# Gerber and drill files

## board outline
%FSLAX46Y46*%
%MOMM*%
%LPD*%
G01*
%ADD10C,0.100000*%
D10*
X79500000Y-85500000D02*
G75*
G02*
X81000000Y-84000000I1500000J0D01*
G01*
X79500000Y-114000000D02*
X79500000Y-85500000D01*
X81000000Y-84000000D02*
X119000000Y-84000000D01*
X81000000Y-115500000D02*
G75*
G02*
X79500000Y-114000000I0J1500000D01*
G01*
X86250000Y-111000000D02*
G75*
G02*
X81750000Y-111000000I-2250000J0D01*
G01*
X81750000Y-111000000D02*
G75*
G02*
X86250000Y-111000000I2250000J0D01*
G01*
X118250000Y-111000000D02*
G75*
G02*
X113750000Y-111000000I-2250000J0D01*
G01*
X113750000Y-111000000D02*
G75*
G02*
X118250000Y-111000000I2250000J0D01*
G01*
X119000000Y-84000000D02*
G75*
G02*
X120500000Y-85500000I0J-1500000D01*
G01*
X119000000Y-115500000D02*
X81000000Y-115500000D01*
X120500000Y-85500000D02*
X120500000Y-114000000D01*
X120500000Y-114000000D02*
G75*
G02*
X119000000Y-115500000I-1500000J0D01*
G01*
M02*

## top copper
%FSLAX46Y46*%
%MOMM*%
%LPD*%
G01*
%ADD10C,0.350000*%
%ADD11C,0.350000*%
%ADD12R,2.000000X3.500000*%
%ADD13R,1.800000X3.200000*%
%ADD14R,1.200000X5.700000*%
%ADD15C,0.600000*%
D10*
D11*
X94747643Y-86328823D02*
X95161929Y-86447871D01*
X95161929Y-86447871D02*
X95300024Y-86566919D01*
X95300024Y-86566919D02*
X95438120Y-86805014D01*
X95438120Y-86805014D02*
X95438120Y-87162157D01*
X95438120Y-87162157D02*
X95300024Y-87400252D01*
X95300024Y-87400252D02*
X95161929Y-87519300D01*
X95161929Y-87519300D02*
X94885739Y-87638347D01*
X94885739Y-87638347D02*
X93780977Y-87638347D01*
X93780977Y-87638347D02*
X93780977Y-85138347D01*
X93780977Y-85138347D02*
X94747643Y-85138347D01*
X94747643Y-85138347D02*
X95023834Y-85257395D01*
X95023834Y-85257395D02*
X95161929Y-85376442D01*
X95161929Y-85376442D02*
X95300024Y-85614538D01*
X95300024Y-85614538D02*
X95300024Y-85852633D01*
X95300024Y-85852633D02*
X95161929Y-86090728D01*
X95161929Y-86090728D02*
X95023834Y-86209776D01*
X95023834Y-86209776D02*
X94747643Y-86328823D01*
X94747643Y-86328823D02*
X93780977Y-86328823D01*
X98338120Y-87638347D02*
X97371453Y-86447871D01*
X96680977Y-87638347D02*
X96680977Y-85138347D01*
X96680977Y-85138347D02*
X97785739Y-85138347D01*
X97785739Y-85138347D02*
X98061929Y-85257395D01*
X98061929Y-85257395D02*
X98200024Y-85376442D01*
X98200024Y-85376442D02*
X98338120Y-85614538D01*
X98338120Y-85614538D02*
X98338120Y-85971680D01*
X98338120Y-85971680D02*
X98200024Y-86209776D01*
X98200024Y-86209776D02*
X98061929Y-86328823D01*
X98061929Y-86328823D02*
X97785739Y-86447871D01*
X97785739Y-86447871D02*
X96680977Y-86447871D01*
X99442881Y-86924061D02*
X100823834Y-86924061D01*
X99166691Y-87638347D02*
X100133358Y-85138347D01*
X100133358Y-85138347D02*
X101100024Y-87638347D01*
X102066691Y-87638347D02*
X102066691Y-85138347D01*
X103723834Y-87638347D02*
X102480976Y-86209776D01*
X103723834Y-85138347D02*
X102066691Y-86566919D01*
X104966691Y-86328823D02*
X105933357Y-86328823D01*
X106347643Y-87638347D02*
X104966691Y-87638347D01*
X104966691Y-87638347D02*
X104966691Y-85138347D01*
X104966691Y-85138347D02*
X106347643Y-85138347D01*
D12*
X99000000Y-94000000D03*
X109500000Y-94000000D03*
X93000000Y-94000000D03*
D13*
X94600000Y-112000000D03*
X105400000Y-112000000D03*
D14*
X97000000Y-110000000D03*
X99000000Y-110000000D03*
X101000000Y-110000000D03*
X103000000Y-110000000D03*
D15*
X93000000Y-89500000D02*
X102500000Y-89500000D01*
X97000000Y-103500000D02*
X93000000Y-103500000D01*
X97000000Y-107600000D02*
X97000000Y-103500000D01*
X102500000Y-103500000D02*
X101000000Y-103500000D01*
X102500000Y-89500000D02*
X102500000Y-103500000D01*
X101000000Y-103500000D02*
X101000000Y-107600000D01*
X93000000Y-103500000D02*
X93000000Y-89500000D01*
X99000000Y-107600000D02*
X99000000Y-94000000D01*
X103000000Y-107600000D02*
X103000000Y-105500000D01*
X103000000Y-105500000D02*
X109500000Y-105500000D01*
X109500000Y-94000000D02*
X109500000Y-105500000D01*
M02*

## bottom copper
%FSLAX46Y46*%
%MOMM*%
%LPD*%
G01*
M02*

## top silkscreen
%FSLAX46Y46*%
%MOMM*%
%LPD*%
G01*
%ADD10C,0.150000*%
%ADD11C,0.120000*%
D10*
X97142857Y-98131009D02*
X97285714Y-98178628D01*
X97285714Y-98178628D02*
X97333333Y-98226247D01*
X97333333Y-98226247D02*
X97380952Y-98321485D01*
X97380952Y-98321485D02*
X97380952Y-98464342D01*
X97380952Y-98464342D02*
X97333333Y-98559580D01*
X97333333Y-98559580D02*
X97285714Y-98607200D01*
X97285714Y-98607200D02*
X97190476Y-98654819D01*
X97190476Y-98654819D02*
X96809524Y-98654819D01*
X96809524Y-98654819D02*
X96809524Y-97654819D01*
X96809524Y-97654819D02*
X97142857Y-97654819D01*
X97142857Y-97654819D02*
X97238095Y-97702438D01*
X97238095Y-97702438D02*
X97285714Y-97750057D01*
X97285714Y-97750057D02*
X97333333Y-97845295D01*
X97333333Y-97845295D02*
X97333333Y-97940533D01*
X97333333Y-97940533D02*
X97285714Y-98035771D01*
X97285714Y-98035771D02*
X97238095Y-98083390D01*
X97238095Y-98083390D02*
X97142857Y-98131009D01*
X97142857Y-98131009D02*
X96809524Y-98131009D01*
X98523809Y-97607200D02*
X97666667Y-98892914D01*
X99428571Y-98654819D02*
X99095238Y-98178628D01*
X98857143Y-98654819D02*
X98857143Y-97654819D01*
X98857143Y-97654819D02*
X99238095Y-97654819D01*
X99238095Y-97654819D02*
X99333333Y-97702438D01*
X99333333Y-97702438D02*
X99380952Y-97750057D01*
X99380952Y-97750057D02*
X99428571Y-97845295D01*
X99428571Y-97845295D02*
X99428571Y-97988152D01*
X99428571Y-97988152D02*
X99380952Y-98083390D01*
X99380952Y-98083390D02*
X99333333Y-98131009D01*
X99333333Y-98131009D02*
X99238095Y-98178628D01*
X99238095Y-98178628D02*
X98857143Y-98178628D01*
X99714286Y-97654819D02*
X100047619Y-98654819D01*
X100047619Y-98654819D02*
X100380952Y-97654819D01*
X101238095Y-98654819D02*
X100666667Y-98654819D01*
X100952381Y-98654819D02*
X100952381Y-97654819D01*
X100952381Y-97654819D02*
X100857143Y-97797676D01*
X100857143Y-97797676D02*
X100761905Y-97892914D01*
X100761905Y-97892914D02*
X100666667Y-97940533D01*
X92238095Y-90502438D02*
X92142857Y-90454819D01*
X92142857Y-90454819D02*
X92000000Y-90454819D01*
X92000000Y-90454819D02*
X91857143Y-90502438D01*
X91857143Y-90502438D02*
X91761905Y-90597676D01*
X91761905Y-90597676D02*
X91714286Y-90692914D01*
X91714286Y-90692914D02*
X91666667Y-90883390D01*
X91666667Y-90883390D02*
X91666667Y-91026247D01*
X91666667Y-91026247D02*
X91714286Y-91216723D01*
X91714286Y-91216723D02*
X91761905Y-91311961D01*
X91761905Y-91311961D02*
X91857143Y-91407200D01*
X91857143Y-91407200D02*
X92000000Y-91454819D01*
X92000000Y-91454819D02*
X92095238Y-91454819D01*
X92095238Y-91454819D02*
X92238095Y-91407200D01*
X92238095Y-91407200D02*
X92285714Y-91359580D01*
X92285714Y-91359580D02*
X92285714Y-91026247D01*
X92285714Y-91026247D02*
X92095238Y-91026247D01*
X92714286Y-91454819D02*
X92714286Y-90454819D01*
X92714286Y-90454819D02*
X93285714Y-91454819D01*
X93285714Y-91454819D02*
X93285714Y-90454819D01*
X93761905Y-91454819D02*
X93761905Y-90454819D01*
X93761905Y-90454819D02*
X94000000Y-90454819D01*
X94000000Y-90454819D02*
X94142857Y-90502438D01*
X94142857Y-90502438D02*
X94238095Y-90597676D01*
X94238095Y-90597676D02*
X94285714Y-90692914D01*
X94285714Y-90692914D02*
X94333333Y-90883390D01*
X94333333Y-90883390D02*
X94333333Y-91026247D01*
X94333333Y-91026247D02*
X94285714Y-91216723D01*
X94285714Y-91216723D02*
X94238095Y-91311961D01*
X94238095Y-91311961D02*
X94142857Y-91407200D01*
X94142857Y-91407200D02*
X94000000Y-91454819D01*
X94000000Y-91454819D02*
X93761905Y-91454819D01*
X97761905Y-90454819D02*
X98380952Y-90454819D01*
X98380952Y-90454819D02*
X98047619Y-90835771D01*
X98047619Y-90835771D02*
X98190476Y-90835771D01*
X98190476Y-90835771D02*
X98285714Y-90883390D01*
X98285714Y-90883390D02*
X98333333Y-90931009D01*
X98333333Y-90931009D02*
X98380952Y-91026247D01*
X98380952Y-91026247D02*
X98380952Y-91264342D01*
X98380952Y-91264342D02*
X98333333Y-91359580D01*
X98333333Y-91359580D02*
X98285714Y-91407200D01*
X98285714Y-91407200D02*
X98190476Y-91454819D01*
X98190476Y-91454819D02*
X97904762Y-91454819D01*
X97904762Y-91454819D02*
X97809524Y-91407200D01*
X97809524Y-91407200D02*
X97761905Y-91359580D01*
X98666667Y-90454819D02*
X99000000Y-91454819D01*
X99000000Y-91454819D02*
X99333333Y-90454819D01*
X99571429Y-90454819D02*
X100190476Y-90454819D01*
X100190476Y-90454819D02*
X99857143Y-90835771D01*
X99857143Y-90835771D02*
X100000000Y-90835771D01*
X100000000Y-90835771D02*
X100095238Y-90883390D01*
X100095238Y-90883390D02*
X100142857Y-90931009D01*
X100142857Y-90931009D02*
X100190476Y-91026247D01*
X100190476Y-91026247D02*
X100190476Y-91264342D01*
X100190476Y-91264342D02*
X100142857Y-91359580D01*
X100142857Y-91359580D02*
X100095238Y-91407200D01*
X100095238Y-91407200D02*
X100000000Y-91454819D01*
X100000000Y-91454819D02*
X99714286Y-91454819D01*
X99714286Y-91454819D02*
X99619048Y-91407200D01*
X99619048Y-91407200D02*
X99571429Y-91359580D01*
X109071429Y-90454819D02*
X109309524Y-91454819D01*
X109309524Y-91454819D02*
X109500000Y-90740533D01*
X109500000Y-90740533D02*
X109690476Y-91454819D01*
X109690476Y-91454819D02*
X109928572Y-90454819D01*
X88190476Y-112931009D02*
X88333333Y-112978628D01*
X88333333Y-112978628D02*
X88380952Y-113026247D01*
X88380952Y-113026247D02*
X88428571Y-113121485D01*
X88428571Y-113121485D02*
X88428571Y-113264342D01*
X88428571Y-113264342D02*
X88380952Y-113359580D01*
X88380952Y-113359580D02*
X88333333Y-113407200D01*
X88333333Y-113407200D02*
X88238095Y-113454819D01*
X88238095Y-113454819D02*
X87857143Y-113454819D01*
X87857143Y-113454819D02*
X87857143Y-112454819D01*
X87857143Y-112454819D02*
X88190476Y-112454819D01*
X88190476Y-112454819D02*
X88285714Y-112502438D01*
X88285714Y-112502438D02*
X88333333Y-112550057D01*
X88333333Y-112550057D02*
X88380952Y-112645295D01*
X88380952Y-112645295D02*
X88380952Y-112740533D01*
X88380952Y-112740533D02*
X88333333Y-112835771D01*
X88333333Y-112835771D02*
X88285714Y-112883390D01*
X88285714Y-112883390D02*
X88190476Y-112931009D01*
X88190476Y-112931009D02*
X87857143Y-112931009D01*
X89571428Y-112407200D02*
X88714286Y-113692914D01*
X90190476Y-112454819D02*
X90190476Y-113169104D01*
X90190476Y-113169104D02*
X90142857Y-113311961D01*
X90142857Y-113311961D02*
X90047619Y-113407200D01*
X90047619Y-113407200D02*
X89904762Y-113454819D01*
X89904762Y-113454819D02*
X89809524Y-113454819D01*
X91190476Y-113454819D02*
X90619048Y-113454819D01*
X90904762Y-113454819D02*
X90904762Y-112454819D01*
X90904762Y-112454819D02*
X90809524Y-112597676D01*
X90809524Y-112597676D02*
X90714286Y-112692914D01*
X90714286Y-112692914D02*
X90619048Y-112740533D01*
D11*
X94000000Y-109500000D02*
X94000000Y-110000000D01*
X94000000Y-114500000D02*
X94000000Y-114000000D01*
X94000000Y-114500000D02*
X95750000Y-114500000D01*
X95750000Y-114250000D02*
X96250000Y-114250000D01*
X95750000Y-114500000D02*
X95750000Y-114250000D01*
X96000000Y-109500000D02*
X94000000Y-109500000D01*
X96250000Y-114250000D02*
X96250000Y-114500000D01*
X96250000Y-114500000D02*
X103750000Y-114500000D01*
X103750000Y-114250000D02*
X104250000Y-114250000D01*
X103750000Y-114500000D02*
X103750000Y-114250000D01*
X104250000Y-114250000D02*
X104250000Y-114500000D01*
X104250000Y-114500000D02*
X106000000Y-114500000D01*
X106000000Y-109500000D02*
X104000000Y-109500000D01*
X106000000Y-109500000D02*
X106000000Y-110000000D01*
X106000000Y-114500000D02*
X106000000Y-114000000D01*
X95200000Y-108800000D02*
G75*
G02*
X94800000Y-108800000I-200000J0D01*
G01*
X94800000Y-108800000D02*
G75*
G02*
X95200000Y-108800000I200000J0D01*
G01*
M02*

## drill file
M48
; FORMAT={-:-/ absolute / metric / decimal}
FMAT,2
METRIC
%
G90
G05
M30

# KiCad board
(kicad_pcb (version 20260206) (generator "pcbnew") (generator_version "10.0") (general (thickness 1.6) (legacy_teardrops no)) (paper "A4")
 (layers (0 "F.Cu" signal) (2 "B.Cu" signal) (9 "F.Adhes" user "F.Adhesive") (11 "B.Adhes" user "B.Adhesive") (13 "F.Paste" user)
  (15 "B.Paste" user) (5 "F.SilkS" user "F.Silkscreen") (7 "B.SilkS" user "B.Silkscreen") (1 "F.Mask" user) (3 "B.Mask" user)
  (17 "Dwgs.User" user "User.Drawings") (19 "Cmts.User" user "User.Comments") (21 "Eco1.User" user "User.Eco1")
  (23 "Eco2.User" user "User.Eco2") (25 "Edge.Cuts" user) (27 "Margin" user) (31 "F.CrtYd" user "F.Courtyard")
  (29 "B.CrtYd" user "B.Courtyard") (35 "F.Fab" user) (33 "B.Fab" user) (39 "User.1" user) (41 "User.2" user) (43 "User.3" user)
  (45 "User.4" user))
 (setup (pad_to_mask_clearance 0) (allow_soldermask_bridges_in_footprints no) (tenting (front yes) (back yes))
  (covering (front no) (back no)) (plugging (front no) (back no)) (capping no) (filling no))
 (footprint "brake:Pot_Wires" (layer "F.Cu") (at 99 94)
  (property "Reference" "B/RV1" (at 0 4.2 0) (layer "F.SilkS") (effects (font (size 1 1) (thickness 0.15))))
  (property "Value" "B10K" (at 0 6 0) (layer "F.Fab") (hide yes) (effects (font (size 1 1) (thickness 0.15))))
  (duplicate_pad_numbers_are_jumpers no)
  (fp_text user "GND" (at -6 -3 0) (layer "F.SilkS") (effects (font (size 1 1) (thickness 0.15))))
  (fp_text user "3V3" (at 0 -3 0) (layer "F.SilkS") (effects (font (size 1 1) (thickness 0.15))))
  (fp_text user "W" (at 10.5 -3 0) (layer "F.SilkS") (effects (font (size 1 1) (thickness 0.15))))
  (pad "1" smd rect (at 0 0) (size 2 3.5) (layers "F.Cu" "F.Mask") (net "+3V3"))
  (pad "2" smd rect (at 10.5 0) (size 2 3.5) (layers "F.Cu" "F.Mask") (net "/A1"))
  (pad "3" smd rect (at -6 0) (size 2 3.5) (layers "F.Cu" "F.Mask") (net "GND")))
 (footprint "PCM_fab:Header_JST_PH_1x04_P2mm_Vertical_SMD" (layer "F.Cu") (at 98 110 90)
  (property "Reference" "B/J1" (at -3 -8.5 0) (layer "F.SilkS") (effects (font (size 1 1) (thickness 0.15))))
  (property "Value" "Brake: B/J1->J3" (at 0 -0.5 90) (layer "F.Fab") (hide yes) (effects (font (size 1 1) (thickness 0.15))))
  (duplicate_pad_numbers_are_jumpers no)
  (fp_line (start 0.5 -4) (end 0 -4) (stroke (width 0.12) (type solid)) (layer "F.SilkS"))
  (fp_line (start -4.5 -4) (end -4 -4) (stroke (width 0.12) (type solid)) (layer "F.SilkS"))
  (fp_line (start -4.5 -4) (end -4.5 -2.25) (stroke (width 0.12) (type solid)) (layer "F.SilkS"))
  (fp_line (start -4.25 -2.25) (end -4.25 -1.75) (stroke (width 0.12) (type solid)) (layer "F.SilkS"))
  (fp_line (start -4.5 -2.25) (end -4.25 -2.25) (stroke (width 0.12) (type solid)) (layer "F.SilkS"))
  (fp_line (start 0.5 -2) (end 0.5 -4) (stroke (width 0.12) (type solid)) (layer "F.SilkS"))
  (fp_line (start -4.25 -1.75) (end -4.5 -1.75) (stroke (width 0.12) (type solid)) (layer "F.SilkS"))
  (fp_line (start -4.5 -1.75) (end -4.5 5.75) (stroke (width 0.12) (type solid)) (layer "F.SilkS"))
  (fp_line (start -4.25 5.75) (end -4.25 6.25) (stroke (width 0.12) (type solid)) (layer "F.SilkS"))
  (fp_line (start -4.5 5.75) (end -4.25 5.75) (stroke (width 0.12) (type solid)) (layer "F.SilkS"))
  (fp_line (start -4.25 6.25) (end -4.5 6.25) (stroke (width 0.12) (type solid)) (layer "F.SilkS"))
  (fp_line (start -4.5 6.25) (end -4.5 8) (stroke (width 0.12) (type solid)) (layer "F.SilkS"))
  (fp_line (start 0.5 8) (end 0.5 6) (stroke (width 0.12) (type solid)) (layer "F.SilkS"))
  (fp_line (start 0.5 8) (end 0 8) (stroke (width 0.12) (type solid)) (layer "F.SilkS"))
  (fp_line (start -4.5 8) (end -4 8) (stroke (width 0.12) (type solid)) (layer "F.SilkS"))
  (fp_circle (center 1.2 -3) (end 1.4 -3) (stroke (width 0.12) (type solid)) (fill no) (layer "F.SilkS"))
  (pad "" smd rect (at -2 -3.4 90) (size 3.2 1.8) (layers "F.Cu" "F.Mask" "F.Paste"))
  (pad "" smd rect (at -2 7.4 90) (size 3.2 1.8) (layers "F.Cu" "F.Mask" "F.Paste"))
  (pad "1" smd rect (at 0 -1 90) (size 5.7 1.2) (layers "F.Cu" "F.Mask" "F.Paste") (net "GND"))
  (pad "2" smd rect (at 0 1 90) (size 5.7 1.2) (layers "F.Cu" "F.Mask" "F.Paste") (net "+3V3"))
  (pad "3" smd rect (at 0 3 90) (size 5.7 1.2) (layers "F.Cu" "F.Mask" "F.Paste") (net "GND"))
  (pad "4" smd rect (at 0 5 90) (size 5.7 1.2) (layers "F.Cu" "F.Mask" "F.Paste") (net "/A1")))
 (gr_arc (start 79.5 85.5) (mid 79.939339 84.439339) (end 81 84) (stroke (width 0.1) (type default)) (layer "Edge.Cuts"))
 (gr_line (start 79.5 114) (end 79.5 85.5) (stroke (width 0.1) (type default)) (layer "Edge.Cuts"))
 (gr_line (start 81 84) (end 119 84) (stroke (width 0.1) (type default)) (layer "Edge.Cuts"))
 (gr_arc (start 81 115.5) (mid 79.939339 115.06066) (end 79.5 114) (stroke (width 0.1) (type default)) (layer "Edge.Cuts"))
 (gr_circle (center 84 111) (end 86.25 111) (stroke (width 0.1) (type default)) (fill no) (layer "Edge.Cuts"))
 (gr_circle (center 116 111) (end 118.25 111) (stroke (width 0.1) (type default)) (fill no) (layer "Edge.Cuts"))
 (gr_arc (start 119 84) (mid 120.06066 84.439339) (end 120.5 85.5) (stroke (width 0.1) (type default)) (layer "Edge.Cuts"))
 (gr_line (start 119 115.5) (end 81 115.5) (stroke (width 0.1) (type default)) (layer "Edge.Cuts"))
 (gr_line (start 120.5 85.5) (end 120.5 114) (stroke (width 0.1) (type default)) (layer "Edge.Cuts"))
 (gr_arc (start 120.5 114) (mid 120.06066 115.06066) (end 119 115.5) (stroke (width 0.1) (type default)) (layer "Edge.Cuts"))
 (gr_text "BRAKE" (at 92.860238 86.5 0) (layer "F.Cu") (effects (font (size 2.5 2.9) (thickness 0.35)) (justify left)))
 (segment (start 93 89.5) (end 102.5 89.5) (width 0.6) (layer "F.Cu") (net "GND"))
 (segment (start 97 103.5) (end 93 103.5) (width 0.6) (layer "F.Cu") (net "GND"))
 (segment (start 97 107.6) (end 97 103.5) (width 0.6) (layer "F.Cu") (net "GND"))
 (segment (start 102.5 103.5) (end 101 103.5) (width 0.6) (layer "F.Cu") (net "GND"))
 (segment (start 102.5 89.5) (end 102.5 103.5) (width 0.6) (layer "F.Cu") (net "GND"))
 (segment (start 101 103.5) (end 101 107.6) (width 0.6) (layer "F.Cu") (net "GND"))
 (segment (start 93 103.5) (end 93 89.5) (width 0.6) (layer "F.Cu") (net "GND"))
 (segment (start 99 107.6) (end 99 94) (width 0.6) (layer "F.Cu") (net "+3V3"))
 (segment (start 103 107.6) (end 103 105.5) (width 0.6) (layer "F.Cu") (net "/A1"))
 (segment (start 103 105.5) (end 109.5 105.5) (width 0.6) (layer "F.Cu") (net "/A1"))
 (segment (start 109.5 94) (end 109.5 105.5) (width 0.6) (layer "F.Cu") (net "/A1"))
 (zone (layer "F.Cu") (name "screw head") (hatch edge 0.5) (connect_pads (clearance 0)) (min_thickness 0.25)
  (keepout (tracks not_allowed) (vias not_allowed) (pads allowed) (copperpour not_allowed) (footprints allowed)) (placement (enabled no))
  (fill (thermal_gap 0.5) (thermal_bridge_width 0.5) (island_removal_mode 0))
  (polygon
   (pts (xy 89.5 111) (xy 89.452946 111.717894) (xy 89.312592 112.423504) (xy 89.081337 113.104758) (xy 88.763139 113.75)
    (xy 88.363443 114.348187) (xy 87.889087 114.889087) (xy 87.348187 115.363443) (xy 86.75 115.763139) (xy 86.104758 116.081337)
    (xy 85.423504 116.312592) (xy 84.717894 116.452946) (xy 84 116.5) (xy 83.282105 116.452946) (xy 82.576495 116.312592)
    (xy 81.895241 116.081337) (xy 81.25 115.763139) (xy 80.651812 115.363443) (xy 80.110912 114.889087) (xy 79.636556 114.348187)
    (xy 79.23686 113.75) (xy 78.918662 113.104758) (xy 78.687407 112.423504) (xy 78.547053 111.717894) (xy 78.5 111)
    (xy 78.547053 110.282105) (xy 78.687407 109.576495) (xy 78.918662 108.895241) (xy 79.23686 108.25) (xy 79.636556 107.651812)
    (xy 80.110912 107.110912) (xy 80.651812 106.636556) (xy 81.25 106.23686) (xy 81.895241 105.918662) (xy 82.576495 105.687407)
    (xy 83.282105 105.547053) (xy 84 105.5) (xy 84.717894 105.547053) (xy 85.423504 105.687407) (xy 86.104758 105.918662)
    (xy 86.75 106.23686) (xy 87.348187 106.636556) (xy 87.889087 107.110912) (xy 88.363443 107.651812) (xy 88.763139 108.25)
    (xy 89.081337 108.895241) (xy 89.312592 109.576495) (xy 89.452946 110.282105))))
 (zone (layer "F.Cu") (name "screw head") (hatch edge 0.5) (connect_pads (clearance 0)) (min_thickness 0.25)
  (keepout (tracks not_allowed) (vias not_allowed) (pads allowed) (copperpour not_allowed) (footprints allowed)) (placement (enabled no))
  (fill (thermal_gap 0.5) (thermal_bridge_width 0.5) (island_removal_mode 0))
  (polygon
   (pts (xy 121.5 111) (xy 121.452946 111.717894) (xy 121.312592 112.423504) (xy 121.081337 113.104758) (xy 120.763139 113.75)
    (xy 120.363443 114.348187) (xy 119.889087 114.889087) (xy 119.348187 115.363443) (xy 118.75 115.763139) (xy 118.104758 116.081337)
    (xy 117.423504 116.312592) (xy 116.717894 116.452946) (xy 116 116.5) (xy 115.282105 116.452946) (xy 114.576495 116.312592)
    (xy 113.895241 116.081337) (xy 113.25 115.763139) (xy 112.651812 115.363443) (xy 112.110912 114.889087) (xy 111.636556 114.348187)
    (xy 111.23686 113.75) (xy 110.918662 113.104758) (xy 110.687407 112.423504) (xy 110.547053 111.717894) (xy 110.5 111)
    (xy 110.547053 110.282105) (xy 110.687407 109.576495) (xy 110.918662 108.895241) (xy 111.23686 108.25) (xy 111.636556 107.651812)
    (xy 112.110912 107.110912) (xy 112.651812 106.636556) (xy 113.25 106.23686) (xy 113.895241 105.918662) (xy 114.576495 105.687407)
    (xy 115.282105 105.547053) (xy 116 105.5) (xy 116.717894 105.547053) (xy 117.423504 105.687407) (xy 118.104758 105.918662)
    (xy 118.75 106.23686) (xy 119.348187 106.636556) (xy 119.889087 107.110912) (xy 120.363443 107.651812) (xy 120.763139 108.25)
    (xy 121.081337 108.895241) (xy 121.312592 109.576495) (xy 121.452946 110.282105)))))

